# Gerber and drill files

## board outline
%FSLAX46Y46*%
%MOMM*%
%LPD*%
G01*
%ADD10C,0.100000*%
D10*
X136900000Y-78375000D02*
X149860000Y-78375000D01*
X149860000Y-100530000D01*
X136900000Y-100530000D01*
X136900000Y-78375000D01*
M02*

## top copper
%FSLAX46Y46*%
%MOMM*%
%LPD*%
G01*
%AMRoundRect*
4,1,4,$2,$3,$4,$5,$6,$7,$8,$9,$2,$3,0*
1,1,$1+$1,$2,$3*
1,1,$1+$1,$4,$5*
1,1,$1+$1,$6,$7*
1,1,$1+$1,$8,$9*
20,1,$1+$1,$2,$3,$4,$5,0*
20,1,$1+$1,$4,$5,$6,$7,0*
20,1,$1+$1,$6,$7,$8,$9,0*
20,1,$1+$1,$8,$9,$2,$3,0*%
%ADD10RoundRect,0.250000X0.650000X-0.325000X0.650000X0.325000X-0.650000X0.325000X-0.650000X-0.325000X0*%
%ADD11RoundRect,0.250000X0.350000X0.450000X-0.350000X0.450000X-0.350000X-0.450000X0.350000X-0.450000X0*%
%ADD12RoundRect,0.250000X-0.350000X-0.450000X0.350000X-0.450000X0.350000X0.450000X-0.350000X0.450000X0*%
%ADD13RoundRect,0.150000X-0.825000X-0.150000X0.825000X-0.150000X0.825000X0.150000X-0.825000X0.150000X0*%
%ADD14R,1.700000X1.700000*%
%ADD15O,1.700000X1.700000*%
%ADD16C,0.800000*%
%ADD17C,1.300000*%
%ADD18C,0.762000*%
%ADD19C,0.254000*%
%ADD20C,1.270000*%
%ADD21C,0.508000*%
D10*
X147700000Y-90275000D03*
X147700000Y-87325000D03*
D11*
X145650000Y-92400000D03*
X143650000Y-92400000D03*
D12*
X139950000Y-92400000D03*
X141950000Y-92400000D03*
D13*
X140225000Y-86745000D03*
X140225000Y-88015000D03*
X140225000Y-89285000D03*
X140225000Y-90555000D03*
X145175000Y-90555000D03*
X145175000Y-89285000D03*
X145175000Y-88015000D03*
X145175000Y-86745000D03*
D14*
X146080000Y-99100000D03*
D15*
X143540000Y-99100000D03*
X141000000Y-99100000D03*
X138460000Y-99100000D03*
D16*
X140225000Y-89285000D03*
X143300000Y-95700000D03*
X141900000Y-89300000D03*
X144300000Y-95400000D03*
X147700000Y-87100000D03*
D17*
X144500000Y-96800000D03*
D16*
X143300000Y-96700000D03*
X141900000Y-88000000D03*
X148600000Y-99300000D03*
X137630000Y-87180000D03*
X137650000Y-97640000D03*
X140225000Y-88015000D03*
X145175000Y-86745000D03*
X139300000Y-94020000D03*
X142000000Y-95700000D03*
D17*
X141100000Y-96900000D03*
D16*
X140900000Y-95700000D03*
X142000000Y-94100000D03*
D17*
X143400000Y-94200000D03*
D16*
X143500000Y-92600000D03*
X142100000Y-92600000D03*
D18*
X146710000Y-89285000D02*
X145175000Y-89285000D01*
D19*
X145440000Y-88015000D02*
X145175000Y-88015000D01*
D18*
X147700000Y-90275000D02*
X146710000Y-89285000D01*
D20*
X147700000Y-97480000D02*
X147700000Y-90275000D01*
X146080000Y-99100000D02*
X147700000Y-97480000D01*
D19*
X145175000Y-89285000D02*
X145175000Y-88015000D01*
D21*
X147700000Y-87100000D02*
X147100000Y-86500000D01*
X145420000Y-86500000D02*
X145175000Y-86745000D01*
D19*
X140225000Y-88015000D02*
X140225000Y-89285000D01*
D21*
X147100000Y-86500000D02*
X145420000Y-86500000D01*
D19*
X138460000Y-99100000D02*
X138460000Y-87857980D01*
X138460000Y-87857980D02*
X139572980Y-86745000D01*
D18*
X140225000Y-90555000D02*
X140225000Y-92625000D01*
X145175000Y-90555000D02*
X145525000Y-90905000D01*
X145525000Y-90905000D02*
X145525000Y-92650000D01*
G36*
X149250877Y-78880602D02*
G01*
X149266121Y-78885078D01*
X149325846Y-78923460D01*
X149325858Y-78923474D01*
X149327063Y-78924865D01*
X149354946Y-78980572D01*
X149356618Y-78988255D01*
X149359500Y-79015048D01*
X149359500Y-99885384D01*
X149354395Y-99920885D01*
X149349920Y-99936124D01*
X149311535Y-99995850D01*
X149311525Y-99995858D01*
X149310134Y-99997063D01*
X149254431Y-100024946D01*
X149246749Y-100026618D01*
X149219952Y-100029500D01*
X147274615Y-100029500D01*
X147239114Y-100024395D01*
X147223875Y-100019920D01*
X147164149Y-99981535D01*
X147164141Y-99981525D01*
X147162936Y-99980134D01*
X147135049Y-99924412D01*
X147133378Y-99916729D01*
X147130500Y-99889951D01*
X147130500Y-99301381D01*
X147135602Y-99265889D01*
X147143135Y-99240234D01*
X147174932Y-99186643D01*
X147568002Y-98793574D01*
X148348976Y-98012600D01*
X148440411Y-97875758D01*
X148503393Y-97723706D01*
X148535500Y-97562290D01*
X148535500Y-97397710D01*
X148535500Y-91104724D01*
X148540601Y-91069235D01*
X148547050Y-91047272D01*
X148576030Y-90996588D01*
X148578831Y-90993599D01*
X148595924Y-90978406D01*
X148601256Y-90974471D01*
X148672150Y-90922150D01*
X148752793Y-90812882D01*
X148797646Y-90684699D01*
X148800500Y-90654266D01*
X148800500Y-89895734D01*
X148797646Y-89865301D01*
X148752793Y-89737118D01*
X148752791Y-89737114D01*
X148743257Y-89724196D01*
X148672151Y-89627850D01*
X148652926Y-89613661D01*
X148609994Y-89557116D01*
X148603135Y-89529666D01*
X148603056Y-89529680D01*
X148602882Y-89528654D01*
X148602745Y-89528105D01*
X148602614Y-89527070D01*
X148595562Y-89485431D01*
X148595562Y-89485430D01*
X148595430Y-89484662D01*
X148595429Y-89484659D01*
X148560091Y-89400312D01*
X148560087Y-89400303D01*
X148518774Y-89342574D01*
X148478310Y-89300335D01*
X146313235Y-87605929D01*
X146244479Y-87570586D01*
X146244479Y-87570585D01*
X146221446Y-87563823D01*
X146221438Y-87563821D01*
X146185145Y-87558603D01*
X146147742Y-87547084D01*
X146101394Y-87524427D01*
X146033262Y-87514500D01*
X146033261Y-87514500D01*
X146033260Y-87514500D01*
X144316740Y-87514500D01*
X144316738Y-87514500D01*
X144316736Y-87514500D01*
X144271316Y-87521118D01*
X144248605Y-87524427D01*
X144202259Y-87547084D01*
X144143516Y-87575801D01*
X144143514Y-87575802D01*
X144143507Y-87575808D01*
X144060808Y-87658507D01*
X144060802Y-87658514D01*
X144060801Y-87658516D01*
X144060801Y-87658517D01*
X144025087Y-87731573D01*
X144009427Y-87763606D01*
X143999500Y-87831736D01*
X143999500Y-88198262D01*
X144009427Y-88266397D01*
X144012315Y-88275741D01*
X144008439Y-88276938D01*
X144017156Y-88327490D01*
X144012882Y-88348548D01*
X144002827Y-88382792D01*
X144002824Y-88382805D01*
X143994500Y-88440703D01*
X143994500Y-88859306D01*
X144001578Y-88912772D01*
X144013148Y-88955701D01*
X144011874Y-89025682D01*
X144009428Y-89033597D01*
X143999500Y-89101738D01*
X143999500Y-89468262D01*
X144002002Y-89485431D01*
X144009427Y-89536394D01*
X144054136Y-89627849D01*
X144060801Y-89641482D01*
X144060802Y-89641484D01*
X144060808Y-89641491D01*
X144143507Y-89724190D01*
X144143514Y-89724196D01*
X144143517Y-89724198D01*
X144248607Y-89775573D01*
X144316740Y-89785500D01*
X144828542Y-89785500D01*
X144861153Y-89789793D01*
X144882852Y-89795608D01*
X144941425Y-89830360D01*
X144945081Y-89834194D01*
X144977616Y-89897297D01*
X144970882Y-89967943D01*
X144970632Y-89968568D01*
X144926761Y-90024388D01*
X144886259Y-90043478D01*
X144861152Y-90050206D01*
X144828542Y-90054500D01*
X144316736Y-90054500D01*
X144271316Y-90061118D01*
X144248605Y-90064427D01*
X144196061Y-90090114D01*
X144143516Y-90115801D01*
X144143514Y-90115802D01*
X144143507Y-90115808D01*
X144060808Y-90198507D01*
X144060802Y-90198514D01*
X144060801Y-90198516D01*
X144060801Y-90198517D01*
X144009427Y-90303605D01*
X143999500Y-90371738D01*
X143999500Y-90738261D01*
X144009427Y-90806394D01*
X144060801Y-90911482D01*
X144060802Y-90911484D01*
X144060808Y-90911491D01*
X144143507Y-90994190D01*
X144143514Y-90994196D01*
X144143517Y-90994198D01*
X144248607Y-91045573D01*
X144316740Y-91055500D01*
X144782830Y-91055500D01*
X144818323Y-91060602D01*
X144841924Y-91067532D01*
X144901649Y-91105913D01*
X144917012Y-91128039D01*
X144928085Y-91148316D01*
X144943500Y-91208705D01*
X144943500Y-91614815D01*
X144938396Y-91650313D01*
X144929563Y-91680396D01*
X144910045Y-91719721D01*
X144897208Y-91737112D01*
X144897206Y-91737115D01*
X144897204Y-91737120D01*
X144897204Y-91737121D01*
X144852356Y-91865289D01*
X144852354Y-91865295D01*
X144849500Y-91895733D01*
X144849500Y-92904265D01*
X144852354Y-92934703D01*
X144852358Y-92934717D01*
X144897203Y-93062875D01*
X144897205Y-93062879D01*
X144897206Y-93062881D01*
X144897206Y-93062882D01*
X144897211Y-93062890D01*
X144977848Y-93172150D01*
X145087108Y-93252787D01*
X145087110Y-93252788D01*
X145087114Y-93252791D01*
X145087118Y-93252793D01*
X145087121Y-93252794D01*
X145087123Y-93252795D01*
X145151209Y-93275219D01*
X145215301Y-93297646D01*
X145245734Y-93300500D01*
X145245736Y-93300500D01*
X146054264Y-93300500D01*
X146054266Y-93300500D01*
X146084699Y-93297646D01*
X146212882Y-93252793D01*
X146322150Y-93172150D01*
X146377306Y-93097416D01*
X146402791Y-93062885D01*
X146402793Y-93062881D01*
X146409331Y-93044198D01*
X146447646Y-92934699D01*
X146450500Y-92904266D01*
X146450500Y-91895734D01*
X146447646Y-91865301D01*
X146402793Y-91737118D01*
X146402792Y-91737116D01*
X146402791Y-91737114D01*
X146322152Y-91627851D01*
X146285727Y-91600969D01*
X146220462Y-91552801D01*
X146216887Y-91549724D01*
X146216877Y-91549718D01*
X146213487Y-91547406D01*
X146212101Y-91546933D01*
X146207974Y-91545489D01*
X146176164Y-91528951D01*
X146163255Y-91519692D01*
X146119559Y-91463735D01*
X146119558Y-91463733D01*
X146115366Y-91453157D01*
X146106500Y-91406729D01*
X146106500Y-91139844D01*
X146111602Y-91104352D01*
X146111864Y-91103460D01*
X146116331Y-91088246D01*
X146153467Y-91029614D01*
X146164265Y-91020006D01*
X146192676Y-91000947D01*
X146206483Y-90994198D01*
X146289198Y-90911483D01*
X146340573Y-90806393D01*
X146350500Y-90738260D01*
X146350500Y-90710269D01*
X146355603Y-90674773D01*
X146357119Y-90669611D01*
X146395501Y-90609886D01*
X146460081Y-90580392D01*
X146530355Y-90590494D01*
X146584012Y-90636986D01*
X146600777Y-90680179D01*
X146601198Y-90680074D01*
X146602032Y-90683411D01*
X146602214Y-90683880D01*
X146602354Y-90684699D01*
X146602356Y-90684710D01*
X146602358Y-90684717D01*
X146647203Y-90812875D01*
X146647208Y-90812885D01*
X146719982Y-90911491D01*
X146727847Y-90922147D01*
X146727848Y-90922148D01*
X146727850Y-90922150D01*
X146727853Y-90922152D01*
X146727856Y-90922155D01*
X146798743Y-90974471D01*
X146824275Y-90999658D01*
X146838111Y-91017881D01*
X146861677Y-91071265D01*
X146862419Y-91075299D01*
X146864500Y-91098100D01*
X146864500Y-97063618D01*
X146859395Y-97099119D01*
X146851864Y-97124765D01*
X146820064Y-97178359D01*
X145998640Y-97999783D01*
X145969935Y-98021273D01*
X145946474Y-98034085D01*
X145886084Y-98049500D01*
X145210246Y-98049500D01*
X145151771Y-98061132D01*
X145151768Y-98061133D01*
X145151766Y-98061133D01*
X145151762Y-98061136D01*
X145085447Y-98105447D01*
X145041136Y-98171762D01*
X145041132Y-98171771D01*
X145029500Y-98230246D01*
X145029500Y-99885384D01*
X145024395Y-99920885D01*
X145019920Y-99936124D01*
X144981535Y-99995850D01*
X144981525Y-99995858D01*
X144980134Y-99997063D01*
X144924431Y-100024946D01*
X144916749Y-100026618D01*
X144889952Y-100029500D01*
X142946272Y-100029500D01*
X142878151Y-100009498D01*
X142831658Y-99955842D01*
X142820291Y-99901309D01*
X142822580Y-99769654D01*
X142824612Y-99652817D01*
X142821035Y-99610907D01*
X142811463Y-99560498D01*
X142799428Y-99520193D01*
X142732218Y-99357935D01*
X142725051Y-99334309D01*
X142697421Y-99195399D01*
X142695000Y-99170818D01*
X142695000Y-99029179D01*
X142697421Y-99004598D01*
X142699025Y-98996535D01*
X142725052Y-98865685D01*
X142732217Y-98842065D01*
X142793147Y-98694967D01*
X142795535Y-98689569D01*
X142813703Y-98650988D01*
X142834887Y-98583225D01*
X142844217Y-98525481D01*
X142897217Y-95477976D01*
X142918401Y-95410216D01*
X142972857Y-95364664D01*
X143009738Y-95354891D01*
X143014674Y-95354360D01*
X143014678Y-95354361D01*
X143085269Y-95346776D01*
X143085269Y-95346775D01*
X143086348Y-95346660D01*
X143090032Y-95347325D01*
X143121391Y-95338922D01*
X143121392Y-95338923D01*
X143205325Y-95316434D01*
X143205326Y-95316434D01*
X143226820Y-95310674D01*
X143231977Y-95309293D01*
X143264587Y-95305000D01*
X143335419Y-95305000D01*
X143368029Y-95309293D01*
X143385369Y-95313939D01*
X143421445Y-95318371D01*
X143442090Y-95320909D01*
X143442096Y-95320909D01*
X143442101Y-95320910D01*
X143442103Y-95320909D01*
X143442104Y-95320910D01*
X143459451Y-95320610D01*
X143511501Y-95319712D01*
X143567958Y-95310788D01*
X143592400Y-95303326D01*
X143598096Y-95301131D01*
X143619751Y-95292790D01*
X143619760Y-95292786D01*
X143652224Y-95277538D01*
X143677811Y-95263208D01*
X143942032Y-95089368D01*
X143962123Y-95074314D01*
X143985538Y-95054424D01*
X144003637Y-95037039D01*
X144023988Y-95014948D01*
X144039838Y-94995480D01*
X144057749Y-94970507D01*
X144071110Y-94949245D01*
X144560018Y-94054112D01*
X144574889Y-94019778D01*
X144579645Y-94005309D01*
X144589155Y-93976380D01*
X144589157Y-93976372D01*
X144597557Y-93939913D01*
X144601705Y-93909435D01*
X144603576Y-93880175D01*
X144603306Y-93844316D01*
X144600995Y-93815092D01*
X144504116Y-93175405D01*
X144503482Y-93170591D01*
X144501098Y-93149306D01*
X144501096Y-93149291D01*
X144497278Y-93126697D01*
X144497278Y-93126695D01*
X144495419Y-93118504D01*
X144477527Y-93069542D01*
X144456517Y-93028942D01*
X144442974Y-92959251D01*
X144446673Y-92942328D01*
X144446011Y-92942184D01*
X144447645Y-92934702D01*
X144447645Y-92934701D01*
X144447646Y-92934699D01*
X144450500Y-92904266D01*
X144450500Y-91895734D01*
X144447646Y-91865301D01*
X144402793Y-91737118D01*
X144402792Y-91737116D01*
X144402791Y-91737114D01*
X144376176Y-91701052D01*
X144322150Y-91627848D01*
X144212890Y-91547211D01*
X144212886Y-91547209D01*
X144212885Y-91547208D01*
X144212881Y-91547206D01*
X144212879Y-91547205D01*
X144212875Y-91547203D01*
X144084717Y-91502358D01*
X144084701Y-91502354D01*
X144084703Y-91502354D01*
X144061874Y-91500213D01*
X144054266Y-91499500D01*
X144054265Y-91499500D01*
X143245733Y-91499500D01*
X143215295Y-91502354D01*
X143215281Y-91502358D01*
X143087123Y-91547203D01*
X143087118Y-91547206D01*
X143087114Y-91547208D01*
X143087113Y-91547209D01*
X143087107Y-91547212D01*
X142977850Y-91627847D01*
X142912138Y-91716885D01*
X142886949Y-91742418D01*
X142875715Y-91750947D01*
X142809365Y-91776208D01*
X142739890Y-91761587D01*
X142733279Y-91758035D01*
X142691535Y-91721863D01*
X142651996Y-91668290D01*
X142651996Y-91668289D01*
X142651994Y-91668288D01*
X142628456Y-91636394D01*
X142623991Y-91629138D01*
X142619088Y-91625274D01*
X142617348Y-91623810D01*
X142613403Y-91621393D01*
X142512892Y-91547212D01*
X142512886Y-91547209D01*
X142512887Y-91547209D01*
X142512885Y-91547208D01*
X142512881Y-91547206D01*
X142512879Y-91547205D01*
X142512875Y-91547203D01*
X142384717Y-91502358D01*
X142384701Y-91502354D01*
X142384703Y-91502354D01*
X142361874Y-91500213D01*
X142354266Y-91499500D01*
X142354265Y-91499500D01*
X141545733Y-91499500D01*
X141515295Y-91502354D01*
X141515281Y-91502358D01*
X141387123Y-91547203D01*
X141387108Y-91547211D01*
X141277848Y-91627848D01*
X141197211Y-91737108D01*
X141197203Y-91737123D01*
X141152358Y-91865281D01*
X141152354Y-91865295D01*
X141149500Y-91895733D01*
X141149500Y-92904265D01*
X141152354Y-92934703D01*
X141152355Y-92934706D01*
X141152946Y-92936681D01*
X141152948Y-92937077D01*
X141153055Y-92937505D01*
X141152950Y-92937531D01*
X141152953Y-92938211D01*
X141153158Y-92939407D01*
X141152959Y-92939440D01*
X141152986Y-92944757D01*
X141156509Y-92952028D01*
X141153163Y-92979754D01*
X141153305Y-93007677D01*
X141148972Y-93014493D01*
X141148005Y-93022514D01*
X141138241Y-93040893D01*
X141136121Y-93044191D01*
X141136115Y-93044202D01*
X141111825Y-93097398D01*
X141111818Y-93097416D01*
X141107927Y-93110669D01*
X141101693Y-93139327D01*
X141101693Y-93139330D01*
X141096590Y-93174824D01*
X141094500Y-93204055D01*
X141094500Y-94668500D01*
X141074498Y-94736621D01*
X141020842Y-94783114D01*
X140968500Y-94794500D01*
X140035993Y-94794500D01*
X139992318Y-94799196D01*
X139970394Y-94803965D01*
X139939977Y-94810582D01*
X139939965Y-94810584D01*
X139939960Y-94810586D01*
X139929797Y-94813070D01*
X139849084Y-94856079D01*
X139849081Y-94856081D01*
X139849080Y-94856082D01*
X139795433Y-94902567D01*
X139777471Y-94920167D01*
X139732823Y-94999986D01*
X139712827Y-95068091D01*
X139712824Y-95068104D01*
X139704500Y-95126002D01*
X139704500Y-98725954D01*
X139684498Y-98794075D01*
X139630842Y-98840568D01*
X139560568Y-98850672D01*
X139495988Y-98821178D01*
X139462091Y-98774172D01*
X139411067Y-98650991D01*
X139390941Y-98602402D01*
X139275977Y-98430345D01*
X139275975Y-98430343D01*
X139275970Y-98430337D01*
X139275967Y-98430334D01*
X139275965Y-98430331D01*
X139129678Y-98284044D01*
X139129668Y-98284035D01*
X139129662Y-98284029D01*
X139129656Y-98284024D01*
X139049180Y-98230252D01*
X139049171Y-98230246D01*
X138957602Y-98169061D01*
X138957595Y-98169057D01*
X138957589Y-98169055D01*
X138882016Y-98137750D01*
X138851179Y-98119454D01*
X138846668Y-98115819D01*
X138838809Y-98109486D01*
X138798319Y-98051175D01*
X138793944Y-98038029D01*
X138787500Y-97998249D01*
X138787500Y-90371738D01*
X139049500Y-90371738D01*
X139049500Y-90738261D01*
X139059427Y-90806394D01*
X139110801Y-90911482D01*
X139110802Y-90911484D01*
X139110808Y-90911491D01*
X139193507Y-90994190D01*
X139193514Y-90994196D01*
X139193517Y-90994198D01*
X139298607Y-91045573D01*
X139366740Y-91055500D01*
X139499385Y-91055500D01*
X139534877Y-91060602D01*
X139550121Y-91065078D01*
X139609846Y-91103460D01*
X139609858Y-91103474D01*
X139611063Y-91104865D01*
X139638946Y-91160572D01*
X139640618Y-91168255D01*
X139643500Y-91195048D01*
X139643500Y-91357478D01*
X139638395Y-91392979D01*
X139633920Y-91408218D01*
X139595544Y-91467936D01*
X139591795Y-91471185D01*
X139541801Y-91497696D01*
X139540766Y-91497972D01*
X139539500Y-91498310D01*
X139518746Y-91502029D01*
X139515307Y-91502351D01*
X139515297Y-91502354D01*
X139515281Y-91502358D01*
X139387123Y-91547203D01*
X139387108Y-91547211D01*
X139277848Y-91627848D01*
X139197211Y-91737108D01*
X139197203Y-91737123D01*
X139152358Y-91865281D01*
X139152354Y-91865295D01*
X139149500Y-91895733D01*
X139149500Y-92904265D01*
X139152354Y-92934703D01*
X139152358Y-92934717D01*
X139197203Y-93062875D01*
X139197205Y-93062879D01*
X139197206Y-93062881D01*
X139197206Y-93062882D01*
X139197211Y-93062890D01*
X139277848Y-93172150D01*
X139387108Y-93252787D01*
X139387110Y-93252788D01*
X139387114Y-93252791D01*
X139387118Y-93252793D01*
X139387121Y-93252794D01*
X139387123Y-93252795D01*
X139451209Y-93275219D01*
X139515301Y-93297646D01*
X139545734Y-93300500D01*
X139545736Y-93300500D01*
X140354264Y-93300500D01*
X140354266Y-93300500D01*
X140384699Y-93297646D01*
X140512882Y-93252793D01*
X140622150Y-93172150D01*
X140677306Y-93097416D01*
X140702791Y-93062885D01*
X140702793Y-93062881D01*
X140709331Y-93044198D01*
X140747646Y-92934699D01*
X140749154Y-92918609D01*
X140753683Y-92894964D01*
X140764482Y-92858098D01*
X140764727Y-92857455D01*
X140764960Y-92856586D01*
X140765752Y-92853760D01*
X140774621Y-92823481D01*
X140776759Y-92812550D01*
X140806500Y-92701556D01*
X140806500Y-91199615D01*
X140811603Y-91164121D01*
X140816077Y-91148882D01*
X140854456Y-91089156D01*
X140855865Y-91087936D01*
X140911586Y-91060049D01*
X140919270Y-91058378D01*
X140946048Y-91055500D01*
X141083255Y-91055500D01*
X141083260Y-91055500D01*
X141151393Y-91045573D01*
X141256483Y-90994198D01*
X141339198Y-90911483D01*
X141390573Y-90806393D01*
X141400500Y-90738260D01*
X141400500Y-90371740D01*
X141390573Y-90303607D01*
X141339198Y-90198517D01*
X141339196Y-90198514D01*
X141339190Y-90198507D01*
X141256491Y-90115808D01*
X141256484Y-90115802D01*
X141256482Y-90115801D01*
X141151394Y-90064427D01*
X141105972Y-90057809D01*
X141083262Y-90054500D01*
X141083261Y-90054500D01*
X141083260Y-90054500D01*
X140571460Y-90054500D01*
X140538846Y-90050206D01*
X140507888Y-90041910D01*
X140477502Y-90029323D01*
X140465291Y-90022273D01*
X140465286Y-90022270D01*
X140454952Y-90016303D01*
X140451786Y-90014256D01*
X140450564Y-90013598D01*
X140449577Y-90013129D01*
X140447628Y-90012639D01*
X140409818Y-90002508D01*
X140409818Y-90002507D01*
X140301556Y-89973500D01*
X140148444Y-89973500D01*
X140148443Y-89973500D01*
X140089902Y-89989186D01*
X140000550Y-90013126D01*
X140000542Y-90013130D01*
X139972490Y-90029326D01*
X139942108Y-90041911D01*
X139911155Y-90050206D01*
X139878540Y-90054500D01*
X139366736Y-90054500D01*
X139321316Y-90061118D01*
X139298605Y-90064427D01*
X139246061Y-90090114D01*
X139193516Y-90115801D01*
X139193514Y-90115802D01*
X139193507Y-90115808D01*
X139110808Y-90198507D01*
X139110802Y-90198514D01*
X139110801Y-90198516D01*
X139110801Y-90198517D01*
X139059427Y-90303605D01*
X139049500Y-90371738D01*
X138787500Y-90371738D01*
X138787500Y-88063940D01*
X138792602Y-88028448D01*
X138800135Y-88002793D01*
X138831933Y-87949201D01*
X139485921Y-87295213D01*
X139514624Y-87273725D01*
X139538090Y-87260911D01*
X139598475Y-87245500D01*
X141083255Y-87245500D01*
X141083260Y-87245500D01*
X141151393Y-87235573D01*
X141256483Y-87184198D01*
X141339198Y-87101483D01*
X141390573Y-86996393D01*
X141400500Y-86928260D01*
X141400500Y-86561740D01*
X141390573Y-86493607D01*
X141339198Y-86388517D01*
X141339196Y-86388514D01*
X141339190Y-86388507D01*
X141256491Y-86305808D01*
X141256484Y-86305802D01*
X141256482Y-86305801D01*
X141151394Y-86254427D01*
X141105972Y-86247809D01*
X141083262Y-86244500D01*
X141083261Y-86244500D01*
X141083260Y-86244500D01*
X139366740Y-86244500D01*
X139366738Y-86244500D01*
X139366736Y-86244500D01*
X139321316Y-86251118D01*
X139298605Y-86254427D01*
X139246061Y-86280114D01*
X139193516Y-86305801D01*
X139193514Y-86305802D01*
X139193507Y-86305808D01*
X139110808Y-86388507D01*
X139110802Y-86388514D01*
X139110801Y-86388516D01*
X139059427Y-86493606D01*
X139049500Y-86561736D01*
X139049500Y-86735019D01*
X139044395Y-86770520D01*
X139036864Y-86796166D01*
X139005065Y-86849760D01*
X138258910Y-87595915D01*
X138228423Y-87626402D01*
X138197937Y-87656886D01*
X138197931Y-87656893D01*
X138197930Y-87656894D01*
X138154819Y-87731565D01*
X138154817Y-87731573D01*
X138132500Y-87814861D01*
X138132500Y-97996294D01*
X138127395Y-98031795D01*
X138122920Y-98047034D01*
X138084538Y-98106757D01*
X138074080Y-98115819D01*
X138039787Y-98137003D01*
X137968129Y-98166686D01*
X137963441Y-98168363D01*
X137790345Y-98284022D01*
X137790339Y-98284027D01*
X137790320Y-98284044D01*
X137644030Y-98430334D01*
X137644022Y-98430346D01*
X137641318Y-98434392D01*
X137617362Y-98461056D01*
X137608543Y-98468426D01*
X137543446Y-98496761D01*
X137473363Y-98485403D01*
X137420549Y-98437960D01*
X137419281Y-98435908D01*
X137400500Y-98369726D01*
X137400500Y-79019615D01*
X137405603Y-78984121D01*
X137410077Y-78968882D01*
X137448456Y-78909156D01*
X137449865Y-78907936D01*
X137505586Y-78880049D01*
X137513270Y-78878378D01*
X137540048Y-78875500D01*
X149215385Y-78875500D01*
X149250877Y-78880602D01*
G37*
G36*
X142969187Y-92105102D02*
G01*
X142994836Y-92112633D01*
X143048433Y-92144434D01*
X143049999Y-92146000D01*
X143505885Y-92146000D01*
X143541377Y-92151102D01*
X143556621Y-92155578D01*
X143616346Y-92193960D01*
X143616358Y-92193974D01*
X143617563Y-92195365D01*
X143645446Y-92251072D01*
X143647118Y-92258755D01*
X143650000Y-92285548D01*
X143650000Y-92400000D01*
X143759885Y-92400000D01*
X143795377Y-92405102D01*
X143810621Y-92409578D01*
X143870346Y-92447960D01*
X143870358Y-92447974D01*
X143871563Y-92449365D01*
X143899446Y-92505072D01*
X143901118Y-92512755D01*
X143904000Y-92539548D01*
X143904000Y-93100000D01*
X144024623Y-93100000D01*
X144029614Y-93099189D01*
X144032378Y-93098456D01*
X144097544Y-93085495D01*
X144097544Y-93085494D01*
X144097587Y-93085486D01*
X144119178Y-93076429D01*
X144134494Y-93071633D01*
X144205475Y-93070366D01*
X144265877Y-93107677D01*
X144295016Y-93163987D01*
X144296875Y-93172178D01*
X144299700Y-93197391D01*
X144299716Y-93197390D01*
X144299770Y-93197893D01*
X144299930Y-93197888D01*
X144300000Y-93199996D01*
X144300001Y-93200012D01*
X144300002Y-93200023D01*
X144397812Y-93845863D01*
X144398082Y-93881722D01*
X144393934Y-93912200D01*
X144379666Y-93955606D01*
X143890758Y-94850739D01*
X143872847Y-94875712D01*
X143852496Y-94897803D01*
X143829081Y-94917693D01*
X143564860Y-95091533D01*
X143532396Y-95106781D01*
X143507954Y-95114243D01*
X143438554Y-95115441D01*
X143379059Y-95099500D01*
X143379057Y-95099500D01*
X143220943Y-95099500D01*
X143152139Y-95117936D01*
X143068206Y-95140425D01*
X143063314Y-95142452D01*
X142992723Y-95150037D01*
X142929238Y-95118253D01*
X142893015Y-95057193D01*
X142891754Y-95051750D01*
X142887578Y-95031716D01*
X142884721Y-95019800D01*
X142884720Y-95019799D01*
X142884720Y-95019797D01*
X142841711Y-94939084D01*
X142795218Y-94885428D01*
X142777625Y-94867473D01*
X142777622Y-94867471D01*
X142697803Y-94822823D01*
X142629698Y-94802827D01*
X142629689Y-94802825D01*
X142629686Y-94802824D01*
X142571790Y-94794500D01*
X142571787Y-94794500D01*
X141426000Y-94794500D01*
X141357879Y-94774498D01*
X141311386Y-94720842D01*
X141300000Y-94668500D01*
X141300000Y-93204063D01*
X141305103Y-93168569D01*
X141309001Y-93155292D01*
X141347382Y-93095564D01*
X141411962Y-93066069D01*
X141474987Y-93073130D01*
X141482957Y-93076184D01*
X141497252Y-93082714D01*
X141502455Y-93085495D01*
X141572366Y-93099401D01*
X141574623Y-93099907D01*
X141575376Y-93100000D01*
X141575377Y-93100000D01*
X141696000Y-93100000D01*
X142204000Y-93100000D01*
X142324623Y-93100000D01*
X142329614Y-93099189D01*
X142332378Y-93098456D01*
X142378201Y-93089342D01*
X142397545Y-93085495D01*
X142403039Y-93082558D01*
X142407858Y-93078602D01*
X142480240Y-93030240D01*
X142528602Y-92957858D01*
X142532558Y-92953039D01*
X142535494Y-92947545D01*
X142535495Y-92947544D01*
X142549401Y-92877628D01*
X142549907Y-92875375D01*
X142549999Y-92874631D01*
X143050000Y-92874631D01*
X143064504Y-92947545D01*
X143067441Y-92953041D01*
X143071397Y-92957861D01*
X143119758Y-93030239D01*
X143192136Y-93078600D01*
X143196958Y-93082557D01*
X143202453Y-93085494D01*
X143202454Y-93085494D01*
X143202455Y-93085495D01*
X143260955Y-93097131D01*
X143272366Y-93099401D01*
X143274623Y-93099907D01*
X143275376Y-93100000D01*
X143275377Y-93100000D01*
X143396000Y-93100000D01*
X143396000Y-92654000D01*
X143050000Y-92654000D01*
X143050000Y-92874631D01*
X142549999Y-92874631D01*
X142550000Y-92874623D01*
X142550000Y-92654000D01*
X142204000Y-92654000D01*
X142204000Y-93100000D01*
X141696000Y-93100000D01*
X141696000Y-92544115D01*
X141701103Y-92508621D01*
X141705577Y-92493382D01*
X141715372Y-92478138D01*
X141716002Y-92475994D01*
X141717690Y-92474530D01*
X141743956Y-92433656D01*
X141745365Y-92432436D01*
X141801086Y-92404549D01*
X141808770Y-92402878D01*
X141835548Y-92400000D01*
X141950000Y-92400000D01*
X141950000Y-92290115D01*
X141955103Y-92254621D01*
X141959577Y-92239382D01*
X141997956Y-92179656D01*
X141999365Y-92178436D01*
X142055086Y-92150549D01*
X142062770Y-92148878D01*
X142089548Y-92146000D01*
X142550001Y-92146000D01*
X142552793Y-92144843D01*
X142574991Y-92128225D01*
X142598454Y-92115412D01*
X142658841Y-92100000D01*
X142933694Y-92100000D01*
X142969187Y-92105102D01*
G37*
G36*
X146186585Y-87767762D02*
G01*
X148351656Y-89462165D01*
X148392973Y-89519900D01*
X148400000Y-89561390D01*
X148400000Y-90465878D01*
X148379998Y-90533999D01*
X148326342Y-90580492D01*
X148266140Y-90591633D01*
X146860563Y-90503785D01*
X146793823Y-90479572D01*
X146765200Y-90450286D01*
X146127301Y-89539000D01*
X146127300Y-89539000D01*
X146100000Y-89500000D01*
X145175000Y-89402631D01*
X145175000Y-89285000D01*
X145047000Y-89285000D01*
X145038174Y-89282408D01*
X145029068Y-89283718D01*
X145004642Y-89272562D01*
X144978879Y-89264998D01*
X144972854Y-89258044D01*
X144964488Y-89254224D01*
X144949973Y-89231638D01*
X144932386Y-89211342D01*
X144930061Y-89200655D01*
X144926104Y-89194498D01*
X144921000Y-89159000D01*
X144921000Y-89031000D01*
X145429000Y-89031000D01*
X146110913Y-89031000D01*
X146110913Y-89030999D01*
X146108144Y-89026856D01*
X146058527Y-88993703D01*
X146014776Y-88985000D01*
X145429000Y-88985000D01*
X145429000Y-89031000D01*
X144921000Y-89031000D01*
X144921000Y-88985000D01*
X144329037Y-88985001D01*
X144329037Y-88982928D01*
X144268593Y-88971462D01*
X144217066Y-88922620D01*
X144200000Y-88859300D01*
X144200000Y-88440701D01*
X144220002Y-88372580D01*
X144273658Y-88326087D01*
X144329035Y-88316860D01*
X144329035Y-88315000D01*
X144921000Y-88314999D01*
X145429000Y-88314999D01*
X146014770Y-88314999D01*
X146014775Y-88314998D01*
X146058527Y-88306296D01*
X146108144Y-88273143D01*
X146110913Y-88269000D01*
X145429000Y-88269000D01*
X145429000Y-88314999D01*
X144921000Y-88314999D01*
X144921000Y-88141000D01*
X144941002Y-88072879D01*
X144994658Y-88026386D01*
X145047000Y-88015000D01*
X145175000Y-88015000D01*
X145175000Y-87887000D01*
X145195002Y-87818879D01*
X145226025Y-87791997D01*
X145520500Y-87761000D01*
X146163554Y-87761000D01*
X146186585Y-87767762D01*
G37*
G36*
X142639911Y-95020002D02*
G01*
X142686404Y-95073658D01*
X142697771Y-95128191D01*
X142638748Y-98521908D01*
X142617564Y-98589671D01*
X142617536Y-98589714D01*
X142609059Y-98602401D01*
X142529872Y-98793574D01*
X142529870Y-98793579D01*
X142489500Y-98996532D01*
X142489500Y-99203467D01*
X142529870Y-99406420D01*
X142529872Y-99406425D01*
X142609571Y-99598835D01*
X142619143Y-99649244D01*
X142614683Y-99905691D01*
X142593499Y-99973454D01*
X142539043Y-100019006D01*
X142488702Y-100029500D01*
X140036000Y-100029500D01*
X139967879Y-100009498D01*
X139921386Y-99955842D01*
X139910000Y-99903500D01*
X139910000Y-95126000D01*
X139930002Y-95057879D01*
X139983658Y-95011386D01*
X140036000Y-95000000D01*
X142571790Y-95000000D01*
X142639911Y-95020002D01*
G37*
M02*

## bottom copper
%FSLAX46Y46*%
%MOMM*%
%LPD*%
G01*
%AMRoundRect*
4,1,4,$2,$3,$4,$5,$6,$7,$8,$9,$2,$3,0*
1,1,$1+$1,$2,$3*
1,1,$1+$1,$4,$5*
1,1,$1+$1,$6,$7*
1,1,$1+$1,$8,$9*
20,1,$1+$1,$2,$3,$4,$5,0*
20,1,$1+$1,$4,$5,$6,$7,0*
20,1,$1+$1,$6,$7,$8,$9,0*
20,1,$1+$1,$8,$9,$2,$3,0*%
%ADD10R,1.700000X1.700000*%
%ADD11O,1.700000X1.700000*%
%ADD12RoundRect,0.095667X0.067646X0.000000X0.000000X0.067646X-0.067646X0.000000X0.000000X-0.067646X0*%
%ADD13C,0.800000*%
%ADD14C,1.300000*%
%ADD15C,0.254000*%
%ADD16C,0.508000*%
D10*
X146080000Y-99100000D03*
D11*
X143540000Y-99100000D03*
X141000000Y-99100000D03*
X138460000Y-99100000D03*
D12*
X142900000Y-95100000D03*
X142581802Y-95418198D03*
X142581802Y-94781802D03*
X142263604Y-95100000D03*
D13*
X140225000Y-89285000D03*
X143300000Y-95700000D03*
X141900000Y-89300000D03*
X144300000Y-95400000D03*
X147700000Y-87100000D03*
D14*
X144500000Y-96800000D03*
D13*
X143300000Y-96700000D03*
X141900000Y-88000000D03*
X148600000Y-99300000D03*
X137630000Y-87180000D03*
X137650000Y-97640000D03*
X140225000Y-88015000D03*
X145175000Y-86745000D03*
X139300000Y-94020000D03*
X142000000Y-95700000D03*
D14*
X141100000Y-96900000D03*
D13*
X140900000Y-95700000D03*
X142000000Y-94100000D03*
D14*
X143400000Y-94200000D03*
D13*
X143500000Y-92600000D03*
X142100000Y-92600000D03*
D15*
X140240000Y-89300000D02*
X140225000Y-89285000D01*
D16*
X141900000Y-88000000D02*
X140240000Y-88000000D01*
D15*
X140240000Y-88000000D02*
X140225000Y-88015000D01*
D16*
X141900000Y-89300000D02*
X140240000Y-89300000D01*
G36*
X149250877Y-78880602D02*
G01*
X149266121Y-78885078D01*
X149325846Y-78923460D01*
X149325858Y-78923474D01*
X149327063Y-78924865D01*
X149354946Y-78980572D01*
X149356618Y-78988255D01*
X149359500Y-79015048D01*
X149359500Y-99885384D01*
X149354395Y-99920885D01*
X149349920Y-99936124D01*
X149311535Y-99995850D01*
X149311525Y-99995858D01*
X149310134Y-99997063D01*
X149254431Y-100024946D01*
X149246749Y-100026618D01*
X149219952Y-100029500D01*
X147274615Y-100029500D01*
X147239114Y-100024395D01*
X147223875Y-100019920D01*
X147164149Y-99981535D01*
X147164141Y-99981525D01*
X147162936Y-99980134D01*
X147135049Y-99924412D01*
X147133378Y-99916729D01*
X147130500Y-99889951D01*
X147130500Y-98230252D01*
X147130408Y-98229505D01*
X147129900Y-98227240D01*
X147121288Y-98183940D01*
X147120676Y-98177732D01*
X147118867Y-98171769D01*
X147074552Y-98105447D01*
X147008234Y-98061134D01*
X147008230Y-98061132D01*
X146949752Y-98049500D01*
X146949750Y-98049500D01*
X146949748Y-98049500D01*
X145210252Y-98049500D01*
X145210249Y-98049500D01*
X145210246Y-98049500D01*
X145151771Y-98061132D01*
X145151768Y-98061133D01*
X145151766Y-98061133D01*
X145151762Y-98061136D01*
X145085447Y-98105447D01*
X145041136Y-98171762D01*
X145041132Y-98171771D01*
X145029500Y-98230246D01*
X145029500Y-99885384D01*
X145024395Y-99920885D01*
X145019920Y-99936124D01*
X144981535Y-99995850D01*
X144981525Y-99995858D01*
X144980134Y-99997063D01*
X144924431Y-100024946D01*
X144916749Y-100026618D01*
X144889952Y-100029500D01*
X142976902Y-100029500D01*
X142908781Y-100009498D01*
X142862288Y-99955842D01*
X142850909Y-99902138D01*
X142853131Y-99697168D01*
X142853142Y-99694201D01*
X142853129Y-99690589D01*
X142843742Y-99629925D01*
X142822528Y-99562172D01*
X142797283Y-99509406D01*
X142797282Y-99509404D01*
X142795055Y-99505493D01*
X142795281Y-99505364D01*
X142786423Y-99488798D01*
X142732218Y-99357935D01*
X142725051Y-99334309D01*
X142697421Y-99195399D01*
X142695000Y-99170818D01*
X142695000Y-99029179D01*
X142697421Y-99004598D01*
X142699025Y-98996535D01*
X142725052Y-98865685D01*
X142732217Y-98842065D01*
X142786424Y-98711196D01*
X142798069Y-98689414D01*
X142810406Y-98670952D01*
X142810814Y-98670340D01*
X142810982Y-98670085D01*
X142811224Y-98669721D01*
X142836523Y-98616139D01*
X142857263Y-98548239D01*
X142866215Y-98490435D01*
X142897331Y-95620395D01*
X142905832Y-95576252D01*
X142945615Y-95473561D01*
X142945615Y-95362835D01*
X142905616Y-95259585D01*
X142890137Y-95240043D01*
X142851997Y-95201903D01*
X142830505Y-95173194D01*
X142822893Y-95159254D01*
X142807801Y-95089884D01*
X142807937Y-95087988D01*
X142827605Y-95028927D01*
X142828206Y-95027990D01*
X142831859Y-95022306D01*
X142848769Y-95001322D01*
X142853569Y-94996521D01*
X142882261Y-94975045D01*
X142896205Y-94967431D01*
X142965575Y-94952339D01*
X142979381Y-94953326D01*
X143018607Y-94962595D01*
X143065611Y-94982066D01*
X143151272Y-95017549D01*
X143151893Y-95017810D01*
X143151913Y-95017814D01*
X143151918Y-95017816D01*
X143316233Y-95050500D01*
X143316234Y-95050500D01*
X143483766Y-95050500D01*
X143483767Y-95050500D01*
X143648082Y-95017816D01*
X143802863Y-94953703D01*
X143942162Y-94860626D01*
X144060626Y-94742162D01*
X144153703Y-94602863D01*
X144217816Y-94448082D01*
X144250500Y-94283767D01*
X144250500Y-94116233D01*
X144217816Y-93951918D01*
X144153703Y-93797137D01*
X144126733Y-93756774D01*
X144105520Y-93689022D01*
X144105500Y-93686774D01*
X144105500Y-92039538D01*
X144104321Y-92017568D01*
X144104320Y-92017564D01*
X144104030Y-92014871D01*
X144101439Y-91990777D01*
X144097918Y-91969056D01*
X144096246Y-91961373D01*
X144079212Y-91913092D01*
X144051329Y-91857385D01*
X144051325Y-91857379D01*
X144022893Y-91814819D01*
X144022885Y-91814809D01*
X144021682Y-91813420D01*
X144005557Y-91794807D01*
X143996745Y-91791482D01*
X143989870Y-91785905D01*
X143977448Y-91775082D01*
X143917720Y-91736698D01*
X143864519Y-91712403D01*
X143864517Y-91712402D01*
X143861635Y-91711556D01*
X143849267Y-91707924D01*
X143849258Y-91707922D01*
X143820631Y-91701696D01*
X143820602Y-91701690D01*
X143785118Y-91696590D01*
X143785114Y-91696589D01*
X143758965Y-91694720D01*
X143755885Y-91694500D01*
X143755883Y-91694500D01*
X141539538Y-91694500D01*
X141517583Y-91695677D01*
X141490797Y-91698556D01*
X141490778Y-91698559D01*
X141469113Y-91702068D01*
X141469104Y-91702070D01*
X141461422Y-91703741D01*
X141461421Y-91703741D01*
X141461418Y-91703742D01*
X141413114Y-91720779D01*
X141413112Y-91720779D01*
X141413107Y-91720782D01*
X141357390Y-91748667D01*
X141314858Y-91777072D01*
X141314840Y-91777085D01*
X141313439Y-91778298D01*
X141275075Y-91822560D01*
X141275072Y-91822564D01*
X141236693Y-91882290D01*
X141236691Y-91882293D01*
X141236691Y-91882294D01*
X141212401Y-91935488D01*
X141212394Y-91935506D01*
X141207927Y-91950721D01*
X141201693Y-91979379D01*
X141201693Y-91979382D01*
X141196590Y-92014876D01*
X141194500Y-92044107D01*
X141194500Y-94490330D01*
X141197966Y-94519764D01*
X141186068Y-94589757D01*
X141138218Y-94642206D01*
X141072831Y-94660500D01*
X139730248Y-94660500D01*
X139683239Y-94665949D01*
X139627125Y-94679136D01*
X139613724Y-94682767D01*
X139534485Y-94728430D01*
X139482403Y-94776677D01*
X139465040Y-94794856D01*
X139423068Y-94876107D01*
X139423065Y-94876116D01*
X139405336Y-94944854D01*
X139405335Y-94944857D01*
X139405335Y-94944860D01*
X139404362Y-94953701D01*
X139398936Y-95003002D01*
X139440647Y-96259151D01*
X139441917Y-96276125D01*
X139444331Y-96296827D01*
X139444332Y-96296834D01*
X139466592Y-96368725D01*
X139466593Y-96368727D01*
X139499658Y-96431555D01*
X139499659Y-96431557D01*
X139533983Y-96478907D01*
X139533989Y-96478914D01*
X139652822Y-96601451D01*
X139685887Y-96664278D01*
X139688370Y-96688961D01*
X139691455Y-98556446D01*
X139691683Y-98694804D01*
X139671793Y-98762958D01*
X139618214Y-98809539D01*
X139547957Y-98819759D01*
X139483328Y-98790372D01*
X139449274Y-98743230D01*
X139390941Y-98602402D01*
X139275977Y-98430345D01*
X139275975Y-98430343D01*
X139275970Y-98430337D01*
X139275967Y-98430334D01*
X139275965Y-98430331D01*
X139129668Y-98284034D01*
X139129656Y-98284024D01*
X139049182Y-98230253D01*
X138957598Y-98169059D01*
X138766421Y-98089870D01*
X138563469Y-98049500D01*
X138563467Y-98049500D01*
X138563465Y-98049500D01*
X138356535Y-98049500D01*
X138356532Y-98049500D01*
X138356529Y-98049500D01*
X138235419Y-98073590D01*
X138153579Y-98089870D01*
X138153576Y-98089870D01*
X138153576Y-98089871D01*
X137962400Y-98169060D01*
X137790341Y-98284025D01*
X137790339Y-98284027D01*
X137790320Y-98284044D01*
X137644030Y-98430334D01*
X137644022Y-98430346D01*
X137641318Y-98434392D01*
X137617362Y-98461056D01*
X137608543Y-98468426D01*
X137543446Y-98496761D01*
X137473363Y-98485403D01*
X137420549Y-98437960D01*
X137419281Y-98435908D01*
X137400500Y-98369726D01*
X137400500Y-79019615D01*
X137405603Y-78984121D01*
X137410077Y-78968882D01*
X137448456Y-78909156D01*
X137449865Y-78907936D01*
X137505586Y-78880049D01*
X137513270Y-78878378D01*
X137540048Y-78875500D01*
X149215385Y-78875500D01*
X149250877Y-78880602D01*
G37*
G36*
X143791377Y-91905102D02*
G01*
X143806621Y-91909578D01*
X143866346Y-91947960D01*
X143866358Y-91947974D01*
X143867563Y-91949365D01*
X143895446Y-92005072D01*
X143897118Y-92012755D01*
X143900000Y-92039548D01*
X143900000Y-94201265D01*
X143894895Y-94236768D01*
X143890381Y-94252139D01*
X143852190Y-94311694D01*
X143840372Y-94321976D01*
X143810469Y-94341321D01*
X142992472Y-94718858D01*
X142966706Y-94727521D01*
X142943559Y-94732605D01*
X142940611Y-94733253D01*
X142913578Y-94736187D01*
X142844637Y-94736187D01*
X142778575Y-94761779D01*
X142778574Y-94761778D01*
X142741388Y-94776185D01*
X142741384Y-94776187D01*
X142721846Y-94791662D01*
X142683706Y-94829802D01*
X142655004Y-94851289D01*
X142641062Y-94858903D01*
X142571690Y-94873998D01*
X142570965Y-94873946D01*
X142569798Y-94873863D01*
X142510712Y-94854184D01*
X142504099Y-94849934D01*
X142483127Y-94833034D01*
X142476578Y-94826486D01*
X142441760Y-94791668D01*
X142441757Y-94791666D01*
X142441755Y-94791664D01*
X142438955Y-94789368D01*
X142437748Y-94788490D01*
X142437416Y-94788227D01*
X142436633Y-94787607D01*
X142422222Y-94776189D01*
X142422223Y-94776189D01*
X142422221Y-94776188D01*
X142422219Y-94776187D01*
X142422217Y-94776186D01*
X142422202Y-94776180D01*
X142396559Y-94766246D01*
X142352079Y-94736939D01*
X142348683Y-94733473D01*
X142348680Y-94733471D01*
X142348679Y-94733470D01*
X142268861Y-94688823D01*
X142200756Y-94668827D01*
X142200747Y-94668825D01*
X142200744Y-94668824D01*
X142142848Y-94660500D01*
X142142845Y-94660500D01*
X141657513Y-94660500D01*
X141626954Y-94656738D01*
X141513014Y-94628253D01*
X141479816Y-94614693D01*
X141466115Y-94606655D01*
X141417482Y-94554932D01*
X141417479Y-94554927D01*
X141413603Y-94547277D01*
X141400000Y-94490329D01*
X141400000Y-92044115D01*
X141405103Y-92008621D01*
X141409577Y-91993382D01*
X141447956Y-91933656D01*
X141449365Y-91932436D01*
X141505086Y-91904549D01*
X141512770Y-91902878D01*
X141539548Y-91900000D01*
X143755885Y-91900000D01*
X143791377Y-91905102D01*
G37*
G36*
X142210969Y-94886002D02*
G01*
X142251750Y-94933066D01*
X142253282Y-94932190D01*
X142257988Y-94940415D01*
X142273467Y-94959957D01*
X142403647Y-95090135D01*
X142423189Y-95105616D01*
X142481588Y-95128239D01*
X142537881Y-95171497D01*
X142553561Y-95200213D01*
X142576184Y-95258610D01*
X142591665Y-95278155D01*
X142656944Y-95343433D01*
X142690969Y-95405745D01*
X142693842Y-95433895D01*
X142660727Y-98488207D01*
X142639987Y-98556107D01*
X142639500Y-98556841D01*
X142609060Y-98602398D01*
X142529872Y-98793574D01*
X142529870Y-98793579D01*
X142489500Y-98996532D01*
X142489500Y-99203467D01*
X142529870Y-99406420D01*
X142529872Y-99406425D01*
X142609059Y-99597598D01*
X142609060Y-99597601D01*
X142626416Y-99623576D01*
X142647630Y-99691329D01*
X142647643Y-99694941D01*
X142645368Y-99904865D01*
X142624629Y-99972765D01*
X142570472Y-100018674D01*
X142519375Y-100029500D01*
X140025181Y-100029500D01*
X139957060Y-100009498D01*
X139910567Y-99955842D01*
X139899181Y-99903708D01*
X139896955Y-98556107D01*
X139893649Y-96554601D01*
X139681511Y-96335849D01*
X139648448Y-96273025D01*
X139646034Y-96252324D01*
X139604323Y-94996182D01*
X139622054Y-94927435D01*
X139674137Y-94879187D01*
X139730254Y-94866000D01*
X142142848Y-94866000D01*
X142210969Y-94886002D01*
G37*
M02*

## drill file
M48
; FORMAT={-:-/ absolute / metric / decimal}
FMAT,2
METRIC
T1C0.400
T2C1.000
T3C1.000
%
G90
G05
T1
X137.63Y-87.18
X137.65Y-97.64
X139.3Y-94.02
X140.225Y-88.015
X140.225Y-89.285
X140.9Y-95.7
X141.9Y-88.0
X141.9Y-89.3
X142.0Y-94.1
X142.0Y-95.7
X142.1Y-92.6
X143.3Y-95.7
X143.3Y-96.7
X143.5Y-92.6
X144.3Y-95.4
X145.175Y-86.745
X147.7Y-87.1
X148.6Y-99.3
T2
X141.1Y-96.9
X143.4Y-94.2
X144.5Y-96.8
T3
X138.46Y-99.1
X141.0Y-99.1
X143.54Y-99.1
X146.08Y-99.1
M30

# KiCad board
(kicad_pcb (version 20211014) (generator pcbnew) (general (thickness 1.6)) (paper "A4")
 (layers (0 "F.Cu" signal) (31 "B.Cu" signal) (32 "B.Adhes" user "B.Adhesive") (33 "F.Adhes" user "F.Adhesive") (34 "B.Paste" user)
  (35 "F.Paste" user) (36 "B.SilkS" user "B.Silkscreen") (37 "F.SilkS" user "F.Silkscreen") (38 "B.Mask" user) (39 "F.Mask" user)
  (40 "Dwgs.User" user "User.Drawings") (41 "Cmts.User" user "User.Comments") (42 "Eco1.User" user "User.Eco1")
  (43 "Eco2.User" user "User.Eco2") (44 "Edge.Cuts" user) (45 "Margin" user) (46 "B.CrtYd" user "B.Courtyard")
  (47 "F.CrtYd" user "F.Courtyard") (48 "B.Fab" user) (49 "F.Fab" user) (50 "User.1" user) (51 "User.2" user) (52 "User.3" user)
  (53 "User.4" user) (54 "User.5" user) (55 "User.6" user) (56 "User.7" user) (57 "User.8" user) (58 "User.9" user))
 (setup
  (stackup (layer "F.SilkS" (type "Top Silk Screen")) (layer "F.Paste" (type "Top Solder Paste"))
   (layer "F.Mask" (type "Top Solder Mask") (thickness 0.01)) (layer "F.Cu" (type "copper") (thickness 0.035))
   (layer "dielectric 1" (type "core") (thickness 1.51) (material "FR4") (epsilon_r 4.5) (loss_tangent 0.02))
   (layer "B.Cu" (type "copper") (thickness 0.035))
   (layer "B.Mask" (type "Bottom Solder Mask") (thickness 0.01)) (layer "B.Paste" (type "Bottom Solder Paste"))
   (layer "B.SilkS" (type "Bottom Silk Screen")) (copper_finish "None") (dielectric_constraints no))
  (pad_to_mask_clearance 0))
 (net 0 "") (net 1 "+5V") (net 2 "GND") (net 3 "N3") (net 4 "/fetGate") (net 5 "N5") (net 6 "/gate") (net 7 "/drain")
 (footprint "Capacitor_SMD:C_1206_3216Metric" (layer "F.Cu") (at 147.7 88.8 90)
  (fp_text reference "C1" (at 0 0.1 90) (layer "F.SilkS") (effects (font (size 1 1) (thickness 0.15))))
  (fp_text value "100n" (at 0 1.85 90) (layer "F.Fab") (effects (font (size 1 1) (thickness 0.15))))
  (pad "1" smd roundrect (at -1.475 0 90) (size 1.15 1.8) (layers "F.Cu" "F.Paste" "F.Mask") (roundrect_rratio 0.2173913043) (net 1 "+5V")
   (zone_connect 2))
  (pad "2" smd roundrect (at 1.475 0 90) (size 1.15 1.8) (layers "F.Cu" "F.Paste" "F.Mask") (roundrect_rratio 0.2173913043) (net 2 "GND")))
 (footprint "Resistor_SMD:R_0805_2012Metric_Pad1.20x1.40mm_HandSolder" (layer "F.Cu") (at 144.65 92.4 180)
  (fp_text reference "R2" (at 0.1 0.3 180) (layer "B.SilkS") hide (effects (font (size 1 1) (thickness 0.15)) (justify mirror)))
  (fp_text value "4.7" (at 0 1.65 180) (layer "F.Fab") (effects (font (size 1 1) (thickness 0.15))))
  (pad "1" smd roundrect (at -1 0 180) (size 1.2 1.4) (layers "F.Cu" "F.Paste" "F.Mask") (roundrect_rratio 0.2083333333) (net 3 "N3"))
  (pad "2" smd roundrect (at 1 0 180) (size 1.2 1.4) (layers "F.Cu" "F.Paste" "F.Mask") (roundrect_rratio 0.2083333333) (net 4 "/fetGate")))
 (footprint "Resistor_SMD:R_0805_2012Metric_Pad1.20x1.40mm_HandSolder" (layer "F.Cu") (at 140.95 92.4)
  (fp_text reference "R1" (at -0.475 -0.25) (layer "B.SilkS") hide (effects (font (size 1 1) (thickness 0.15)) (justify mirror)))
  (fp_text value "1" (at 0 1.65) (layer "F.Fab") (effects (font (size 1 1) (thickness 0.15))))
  (pad "1" smd roundrect (at -1 0) (size 1.2 1.4) (layers "F.Cu" "F.Paste" "F.Mask") (roundrect_rratio 0.2083333333) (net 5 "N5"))
  (pad "2" smd roundrect (at 1 0) (size 1.2 1.4) (layers "F.Cu" "F.Paste" "F.Mask") (roundrect_rratio 0.2083333333) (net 4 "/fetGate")))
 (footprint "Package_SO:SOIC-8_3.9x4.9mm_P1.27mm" (layer "F.Cu") (at 142.7 88.65)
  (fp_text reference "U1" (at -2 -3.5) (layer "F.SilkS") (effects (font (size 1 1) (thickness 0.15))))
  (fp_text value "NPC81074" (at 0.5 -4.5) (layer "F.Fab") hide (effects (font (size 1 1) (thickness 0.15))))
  (pad "1" smd roundrect (at -2.475 -1.905) (size 1.95 0.6) (layers "F.Cu" "F.Paste" "F.Mask") (roundrect_rratio 0.25) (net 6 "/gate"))
  (pad "2" smd roundrect (at -2.475 -0.635) (size 1.95 0.6) (layers "F.Cu" "F.Paste" "F.Mask") (roundrect_rratio 0.25) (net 2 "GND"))
  (pad "3" smd roundrect (at -2.475 0.635) (size 1.95 0.6) (layers "F.Cu" "F.Paste" "F.Mask") (roundrect_rratio 0.25) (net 2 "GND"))
  (pad "4" smd roundrect (at -2.475 1.905) (size 1.95 0.6) (layers "F.Cu" "F.Paste" "F.Mask") (roundrect_rratio 0.25) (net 5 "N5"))
  (pad "5" smd roundrect (at 2.475 1.905) (size 1.95 0.6) (layers "F.Cu" "F.Paste" "F.Mask") (roundrect_rratio 0.25) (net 3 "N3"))
  (pad "6" smd roundrect (at 2.475 0.635) (size 1.95 0.6) (layers "F.Cu" "F.Paste" "F.Mask") (roundrect_rratio 0.25) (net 1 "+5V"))
  (pad "7" smd roundrect (at 2.475 -0.635) (size 1.95 0.6) (layers "F.Cu" "F.Paste" "F.Mask") (roundrect_rratio 0.25) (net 1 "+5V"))
  (pad "8" smd roundrect (at 2.475 -1.905) (size 1.95 0.6) (layers "F.Cu" "F.Paste" "F.Mask") (roundrect_rratio 0.25) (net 2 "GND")))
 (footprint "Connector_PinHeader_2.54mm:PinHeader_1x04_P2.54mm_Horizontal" (layer "F.Cu") (at 146.08 99.1 -90)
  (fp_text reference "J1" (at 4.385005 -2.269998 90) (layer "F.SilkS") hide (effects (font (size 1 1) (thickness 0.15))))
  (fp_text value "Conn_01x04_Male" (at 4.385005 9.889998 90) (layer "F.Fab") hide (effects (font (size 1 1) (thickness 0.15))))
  (pad "1" thru_hole rect (at 0 0 270) (size 1.7 1.7) (drill 1) (layers *.Cu *.Mask) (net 1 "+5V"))
  (pad "2" thru_hole oval (at 0 2.54 270) (size 1.7 1.7) (drill 1) (layers *.Cu *.Mask) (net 2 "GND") (zone_connect 2))
  (pad "3" thru_hole oval (at 0 5.08 270) (size 1.7 1.7) (drill 1) (layers *.Cu *.Mask) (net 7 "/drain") (zone_connect 2))
  (pad "4" thru_hole oval (at 0 7.62 270) (size 1.7 1.7) (drill 1) (layers *.Cu *.Mask) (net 6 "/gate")))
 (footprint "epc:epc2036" (layer "B.Cu") (at 143.218198 95.1 135)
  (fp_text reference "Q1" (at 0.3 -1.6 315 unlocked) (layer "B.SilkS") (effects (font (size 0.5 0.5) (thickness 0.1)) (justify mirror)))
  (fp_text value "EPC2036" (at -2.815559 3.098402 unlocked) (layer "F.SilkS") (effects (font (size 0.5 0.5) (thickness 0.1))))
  (pad "1" smd roundrect (at 0.225 -0.225 135) (size 0.287 0.287) (layers "B.Cu" "B.Paste") (roundrect_rratio 0.3333344948) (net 2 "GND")
   (solder_mask_margin -0.05) (solder_paste_margin -0.025) (zone_connect 2))
  (pad "2" smd roundrect (at 0.225 -0.675 135) (size 0.287 0.287) (layers "B.Cu" "B.Paste") (roundrect_rratio 0.3333344948) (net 7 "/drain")
   (solder_mask_margin -0.05) (solder_paste_margin -0.025) (zone_connect 2))
  (pad "3" smd roundrect (at 0.675 -0.225 135) (size 0.287 0.287) (layers "B.Cu" "B.Paste") (roundrect_rratio 0.3333344948)
   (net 4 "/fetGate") (solder_mask_margin -0.05) (solder_paste_margin -0.025) (zone_connect 2))
  (pad "4" smd roundrect (at 0.675 -0.675 135) (size 0.287 0.287) (layers "B.Cu" "B.Paste") (roundrect_rratio 0.3333344948) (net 7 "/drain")
   (solder_mask_margin -0.05) (solder_paste_margin -0.025) (zone_connect 2)))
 (gr_rect (start 149.86 78.375) (end 136.9 100.53) (layer "Edge.Cuts") (width 0.1) (fill none))
 (segment (start 146.71 89.285) (end 145.175 89.285) (width 0.762) (layer "F.Cu") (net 1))
 (segment (start 145.44 88.015) (end 145.175 88.015) (width 0.254) (layer "F.Cu") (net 1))
 (segment (start 147.7 90.275) (end 146.71 89.285) (width 0.762) (layer "F.Cu") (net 1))
 (segment (start 147.7 97.48) (end 147.7 90.275) (width 1.27) (layer "F.Cu") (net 1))
 (segment (start 146.08 99.1) (end 147.7 97.48) (width 1.27) (layer "F.Cu") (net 1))
 (segment (start 145.175 89.285) (end 145.175 88.015) (width 0.254) (layer "F.Cu") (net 1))
 (segment (start 147.7 87.1) (end 147.1 86.5) (width 0.508) (layer "F.Cu") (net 2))
 (segment (start 145.42 86.5) (end 145.175 86.745) (width 0.508) (layer "F.Cu") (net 2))
 (segment (start 140.225 88.015) (end 140.225 89.285) (width 0.254) (layer "F.Cu") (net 2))
 (segment (start 147.1 86.5) (end 145.42 86.5) (width 0.508) (layer "F.Cu") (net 2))
 (via (at 140.225 89.285) (size 0.8) (drill 0.4) (layers "F.Cu" "B.Cu") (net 2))
 (via (at 143.3 95.7) (size 0.8) (drill 0.4) (layers "F.Cu" "B.Cu") (free) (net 2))
 (via (at 141.9 89.3) (size 0.8) (drill 0.4) (layers "F.Cu" "B.Cu") (free) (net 2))
 (via (at 144.3 95.4) (size 0.8) (drill 0.4) (layers "F.Cu" "B.Cu") (free) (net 2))
 (via (at 147.7 87.1) (size 0.8) (drill 0.4) (layers "F.Cu" "B.Cu") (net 2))
 (via (at 144.5 96.8) (size 1.3) (drill 1) (layers "F.Cu" "B.Cu") (free) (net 2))
 (via (at 143.3 96.7) (size 0.8) (drill 0.4) (layers "F.Cu" "B.Cu") (free) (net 2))
 (via (at 141.9 88) (size 0.8) (drill 0.4) (layers "F.Cu" "B.Cu") (free) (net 2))
 (via (at 148.6 99.3) (size 0.8) (drill 0.4) (layers "F.Cu" "B.Cu") (free) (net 2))
 (via (at 137.63 87.18) (size 0.8) (drill 0.4) (layers "F.Cu" "B.Cu") (free) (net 2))
 (via (at 137.65 97.64) (size 0.8) (drill 0.4) (layers "F.Cu" "B.Cu") (free) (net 2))
 (via (at 140.225 88.015) (size 0.8) (drill 0.4) (layers "F.Cu" "B.Cu") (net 2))
 (via (at 145.175 86.745) (size 0.8) (drill 0.4) (layers "F.Cu" "B.Cu") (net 2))
 (via (at 139.3 94.02) (size 0.8) (drill 0.4) (layers "F.Cu" "B.Cu") (free) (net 2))
 (segment (start 140.24 89.3) (end 140.225 89.285) (width 0.254) (layer "B.Cu") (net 2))
 (segment (start 141.9 88) (end 140.24 88) (width 0.508) (layer "B.Cu") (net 2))
 (segment (start 140.24 88) (end 140.225 88.015) (width 0.254) (layer "B.Cu") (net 2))
 (segment (start 141.9 89.3) (end 140.24 89.3) (width 0.508) (layer "B.Cu") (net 2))
 (segment (start 138.46 99.1) (end 138.46 87.85798) (width 0.254) (layer "F.Cu") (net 6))
 (segment (start 138.46 87.85798) (end 139.57298 86.745) (width 0.254) (layer "F.Cu") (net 6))
 (via (at 142 95.7) (size 0.8) (drill 0.4) (layers "F.Cu" "B.Cu") (free) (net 7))
 (via (at 141.1 96.9) (size 1.3) (drill 1) (layers "F.Cu" "B.Cu") (free) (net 7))
 (via (at 140.9 95.7) (size 0.8) (drill 0.4) (layers "F.Cu" "B.Cu") (free) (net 7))
 (segment (start 140.225 90.555) (end 140.225 92.625) (width 0.762) (layer "F.Cu") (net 5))
 (segment (start 145.175 90.555) (end 145.525 90.905) (width 0.762) (layer "F.Cu") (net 3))
 (segment (start 145.525 90.905) (end 145.525 92.65) (width 0.762) (layer "F.Cu") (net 3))
 (via (at 142 94.1) (size 0.8) (drill 0.4) (layers "F.Cu" "B.Cu") (free) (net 4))
 (via (at 143.4 94.2) (size 1.3) (drill 1) (layers "F.Cu" "B.Cu") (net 4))
 (via (at 143.5 92.6) (size 0.8) (drill 0.4) (layers "F.Cu" "B.Cu") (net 4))
 (via (at 142.1 92.6) (size 0.8) (drill 0.4) (layers "F.Cu" "B.Cu") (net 4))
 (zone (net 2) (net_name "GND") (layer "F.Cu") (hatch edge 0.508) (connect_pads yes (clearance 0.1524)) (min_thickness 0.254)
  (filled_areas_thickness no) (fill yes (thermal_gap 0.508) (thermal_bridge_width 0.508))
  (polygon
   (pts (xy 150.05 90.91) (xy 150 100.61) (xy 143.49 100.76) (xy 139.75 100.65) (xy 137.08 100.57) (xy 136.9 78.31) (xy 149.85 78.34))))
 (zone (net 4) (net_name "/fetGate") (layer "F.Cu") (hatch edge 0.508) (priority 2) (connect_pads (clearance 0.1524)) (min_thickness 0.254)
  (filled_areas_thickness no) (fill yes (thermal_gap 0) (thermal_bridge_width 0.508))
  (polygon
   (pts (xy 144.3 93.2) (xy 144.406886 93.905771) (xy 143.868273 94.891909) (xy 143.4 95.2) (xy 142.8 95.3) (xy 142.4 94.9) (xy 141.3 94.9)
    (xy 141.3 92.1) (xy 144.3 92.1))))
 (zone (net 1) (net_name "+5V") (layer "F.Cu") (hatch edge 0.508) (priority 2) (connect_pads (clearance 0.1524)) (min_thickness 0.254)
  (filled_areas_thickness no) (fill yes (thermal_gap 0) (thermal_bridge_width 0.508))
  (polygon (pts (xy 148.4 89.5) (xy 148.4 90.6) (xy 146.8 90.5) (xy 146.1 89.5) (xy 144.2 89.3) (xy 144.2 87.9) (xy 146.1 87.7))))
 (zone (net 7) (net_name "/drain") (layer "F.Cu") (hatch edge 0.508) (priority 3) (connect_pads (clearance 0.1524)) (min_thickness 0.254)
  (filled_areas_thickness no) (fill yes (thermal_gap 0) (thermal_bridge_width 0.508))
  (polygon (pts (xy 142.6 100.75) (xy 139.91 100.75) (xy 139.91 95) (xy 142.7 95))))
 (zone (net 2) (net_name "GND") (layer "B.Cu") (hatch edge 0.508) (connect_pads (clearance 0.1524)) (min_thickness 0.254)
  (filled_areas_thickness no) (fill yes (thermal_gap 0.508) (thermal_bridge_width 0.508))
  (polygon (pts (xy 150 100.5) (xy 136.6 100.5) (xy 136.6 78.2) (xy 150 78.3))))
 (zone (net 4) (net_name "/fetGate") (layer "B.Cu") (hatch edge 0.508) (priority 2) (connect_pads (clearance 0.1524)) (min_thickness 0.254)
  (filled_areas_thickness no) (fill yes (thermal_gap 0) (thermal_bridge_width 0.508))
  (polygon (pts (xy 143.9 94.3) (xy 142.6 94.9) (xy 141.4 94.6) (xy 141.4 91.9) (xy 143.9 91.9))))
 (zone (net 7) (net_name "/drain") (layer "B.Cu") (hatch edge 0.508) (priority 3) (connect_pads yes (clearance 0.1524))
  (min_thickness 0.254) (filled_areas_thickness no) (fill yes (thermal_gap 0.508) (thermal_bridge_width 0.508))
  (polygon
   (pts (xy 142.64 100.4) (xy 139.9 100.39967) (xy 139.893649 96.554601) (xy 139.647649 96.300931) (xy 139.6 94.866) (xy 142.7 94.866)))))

